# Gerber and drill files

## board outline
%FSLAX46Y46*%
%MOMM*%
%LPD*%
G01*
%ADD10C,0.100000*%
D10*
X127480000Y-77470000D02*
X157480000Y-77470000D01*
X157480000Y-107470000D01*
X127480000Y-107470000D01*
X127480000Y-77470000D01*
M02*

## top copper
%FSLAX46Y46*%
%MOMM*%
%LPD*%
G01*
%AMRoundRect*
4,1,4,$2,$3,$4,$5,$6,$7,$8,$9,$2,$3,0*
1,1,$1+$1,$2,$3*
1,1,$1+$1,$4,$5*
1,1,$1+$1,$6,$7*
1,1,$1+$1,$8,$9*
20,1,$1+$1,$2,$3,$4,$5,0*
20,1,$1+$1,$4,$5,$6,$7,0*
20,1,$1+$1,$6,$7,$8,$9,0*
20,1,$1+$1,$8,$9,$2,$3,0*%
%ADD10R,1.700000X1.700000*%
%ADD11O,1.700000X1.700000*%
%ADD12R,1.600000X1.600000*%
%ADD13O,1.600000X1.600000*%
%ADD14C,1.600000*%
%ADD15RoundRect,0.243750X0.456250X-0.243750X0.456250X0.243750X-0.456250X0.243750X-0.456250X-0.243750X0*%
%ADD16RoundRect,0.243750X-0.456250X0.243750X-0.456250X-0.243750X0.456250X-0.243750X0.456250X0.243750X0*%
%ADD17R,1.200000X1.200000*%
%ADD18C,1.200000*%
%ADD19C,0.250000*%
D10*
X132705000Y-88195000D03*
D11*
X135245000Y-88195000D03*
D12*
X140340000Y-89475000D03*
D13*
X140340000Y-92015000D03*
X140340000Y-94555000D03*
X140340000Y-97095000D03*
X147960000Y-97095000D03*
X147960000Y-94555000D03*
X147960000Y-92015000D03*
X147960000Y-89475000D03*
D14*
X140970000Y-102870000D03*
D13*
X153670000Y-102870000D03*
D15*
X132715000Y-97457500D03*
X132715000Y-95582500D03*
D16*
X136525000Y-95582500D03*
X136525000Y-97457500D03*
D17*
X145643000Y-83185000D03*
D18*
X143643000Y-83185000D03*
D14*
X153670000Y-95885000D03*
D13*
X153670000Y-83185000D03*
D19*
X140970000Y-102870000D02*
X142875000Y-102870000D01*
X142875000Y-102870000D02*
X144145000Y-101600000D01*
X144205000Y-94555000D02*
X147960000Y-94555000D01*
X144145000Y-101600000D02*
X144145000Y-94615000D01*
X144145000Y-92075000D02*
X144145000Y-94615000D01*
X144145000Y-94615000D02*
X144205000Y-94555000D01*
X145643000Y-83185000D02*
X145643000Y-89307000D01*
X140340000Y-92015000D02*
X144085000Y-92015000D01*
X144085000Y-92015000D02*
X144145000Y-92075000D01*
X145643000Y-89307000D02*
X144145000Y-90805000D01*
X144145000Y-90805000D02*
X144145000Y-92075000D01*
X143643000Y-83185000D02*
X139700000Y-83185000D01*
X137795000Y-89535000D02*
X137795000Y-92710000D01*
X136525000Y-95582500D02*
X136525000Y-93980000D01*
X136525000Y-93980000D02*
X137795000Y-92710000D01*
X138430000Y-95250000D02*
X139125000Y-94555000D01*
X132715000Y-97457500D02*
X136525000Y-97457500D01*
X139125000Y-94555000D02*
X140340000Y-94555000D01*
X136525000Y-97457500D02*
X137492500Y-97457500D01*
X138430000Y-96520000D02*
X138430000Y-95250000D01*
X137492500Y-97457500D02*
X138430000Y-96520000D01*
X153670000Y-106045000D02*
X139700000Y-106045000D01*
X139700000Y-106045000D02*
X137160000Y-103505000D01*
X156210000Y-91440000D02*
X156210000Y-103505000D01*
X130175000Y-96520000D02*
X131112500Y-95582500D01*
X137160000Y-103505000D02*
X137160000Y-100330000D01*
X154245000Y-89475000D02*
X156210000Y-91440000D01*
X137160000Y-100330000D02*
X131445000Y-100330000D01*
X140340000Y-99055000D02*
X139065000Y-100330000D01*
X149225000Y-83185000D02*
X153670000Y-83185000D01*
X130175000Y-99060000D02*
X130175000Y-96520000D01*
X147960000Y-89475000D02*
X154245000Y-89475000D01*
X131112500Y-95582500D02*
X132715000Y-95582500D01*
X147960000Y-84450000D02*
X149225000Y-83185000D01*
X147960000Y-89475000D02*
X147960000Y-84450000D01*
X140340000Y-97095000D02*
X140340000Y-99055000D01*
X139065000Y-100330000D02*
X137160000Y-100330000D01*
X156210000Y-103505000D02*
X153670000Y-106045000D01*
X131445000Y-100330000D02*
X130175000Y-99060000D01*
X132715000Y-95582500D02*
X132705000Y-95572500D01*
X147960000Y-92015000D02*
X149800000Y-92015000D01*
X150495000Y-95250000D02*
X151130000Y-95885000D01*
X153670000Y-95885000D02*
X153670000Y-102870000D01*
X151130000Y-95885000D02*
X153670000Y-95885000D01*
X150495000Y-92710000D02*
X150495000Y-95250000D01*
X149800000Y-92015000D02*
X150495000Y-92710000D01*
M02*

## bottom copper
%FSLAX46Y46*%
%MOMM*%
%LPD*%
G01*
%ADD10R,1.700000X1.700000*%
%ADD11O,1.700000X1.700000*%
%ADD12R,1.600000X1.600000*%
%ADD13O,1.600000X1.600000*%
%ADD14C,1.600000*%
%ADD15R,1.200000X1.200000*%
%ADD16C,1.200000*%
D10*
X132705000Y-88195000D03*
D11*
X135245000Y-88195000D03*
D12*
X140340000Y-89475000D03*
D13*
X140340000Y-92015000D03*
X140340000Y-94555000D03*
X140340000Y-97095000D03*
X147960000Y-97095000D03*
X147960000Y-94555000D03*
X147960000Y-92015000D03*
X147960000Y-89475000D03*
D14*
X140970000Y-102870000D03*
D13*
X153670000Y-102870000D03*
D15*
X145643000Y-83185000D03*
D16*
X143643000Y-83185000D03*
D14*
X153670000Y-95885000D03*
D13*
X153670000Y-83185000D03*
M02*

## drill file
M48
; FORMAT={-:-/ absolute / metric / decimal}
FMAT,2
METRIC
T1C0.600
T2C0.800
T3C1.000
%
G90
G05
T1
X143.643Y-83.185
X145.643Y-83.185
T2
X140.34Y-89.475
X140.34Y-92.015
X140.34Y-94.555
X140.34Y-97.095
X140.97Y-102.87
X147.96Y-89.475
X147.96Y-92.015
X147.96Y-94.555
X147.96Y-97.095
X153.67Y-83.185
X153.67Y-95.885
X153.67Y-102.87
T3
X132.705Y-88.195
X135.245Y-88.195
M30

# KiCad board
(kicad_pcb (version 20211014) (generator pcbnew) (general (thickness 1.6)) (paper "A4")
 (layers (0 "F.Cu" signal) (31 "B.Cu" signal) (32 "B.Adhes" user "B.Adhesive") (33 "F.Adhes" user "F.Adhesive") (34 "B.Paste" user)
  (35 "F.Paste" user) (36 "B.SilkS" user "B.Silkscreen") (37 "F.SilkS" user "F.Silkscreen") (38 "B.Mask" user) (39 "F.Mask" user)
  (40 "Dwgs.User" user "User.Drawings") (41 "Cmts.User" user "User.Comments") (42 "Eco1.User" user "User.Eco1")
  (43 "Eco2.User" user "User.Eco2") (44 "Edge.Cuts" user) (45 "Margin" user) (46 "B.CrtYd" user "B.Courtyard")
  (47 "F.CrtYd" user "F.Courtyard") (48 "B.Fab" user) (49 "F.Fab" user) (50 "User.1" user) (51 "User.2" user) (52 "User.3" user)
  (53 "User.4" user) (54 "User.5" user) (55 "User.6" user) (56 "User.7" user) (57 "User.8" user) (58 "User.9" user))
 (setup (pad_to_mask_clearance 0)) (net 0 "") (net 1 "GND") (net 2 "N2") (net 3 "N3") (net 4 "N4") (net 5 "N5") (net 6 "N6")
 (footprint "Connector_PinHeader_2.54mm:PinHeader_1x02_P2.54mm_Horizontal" (layer "F.Cu") (at 132.705 88.195 90)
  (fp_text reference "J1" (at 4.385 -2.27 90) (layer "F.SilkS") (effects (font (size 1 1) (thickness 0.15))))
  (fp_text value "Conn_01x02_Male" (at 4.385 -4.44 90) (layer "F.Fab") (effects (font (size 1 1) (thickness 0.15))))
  (pad "1" thru_hole rect (at 0 0 90) (size 1.7 1.7) (drill 1) (layers *.Cu *.Mask) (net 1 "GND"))
  (pad "2" thru_hole oval (at 0 2.54 90) (size 1.7 1.7) (drill 1) (layers *.Cu *.Mask) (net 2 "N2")))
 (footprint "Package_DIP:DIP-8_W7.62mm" (layer "F.Cu") (at 140.34 89.475)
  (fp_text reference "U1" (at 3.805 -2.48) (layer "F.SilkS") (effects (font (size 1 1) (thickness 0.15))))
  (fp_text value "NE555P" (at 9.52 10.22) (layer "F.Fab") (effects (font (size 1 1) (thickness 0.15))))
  (pad "1" thru_hole rect (at 0 0) (size 1.6 1.6) (drill 0.8) (layers *.Cu *.Mask) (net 1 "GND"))
  (pad "2" thru_hole oval (at 0 2.54) (size 1.6 1.6) (drill 0.8) (layers *.Cu *.Mask) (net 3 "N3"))
  (pad "3" thru_hole oval (at 0 5.08) (size 1.6 1.6) (drill 0.8) (layers *.Cu *.Mask) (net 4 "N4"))
  (pad "4" thru_hole oval (at 0 7.62) (size 1.6 1.6) (drill 0.8) (layers *.Cu *.Mask) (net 2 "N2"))
  (pad "5" thru_hole oval (at 7.62 7.62) (size 1.6 1.6) (drill 0.8) (layers *.Cu *.Mask) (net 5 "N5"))
  (pad "6" thru_hole oval (at 7.62 5.08) (size 1.6 1.6) (drill 0.8) (layers *.Cu *.Mask) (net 3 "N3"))
  (pad "7" thru_hole oval (at 7.62 2.54) (size 1.6 1.6) (drill 0.8) (layers *.Cu *.Mask) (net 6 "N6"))
  (pad "8" thru_hole oval (at 7.62 0) (size 1.6 1.6) (drill 0.8) (layers *.Cu *.Mask) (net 2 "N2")))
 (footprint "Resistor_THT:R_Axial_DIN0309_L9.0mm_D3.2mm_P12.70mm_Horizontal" (layer "F.Cu") (at 140.97 102.87)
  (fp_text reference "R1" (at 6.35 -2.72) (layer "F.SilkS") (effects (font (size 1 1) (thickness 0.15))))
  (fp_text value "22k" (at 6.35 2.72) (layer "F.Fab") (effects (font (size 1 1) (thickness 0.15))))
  (pad "1" thru_hole circle (at 0 0) (size 1.6 1.6) (drill 0.8) (layers *.Cu *.Mask) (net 3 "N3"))
  (pad "2" thru_hole oval (at 12.7 0) (size 1.6 1.6) (drill 0.8) (layers *.Cu *.Mask) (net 6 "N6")))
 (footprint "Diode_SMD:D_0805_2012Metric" (layer "F.Cu") (at 132.715 96.52 90)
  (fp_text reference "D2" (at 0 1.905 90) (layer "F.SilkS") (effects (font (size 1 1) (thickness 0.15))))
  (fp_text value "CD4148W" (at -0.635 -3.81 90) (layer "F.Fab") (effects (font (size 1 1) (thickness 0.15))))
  (pad "1" smd roundrect (at -0.9375 0 90) (size 0.975 1.4) (layers "F.Cu" "F.Paste" "F.Mask") (roundrect_rratio 0.25) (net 4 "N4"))
  (pad "2" smd roundrect (at 0.9375 0 90) (size 0.975 1.4) (layers "F.Cu" "F.Paste" "F.Mask") (roundrect_rratio 0.25) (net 2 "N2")))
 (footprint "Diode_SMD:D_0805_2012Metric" (layer "F.Cu") (at 136.525 96.52 -90)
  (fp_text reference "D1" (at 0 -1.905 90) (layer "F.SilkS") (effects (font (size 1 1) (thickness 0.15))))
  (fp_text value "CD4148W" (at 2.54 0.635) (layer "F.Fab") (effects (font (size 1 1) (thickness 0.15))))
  (pad "1" smd roundrect (at -0.9375 0 270) (size 0.975 1.4) (layers "F.Cu" "F.Paste" "F.Mask") (roundrect_rratio 0.25) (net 1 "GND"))
  (pad "2" smd roundrect (at 0.9375 0 270) (size 0.975 1.4) (layers "F.Cu" "F.Paste" "F.Mask") (roundrect_rratio 0.25) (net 4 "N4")))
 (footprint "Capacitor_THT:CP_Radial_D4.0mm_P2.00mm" (layer "F.Cu") (at 145.643 83.185 180)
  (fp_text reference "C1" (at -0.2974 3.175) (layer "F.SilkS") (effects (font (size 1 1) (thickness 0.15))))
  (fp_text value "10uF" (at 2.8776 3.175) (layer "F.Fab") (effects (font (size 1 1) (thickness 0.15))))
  (pad "1" thru_hole rect (at 0 0 180) (size 1.2 1.2) (drill 0.6) (layers *.Cu *.Mask) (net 3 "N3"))
  (pad "2" thru_hole circle (at 2 0 180) (size 1.2 1.2) (drill 0.6) (layers *.Cu *.Mask) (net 1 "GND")))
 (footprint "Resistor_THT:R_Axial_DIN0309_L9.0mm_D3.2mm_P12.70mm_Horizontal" (layer "F.Cu") (at 153.67 95.885 90)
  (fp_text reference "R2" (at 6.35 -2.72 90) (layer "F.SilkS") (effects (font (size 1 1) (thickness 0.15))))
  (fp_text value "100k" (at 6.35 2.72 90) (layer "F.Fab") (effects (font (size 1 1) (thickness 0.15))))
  (pad "1" thru_hole circle (at 0 0 90) (size 1.6 1.6) (drill 0.8) (layers *.Cu *.Mask) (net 6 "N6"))
  (pad "2" thru_hole oval (at 12.7 0 90) (size 1.6 1.6) (drill 0.8) (layers *.Cu *.Mask) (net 2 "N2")))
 (gr_rect (start 127.48 77.47) (end 157.48 107.47) (layer "Edge.Cuts") (width 0.1) (fill none))
 (segment (start 140.97 102.87) (end 142.875 102.87) (width 0.25) (layer "F.Cu") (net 3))
 (segment (start 142.875 102.87) (end 144.145 101.6) (width 0.25) (layer "F.Cu") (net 3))
 (segment (start 144.205 94.555) (end 147.96 94.555) (width 0.25) (layer "F.Cu") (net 3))
 (segment (start 144.145 101.6) (end 144.145 94.615) (width 0.25) (layer "F.Cu") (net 3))
 (segment (start 144.145 92.075) (end 144.145 94.615) (width 0.25) (layer "F.Cu") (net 3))
 (segment (start 144.145 94.615) (end 144.205 94.555) (width 0.25) (layer "F.Cu") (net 3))
 (segment (start 145.643 83.185) (end 145.643 89.307) (width 0.25) (layer "F.Cu") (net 3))
 (segment (start 140.34 92.015) (end 144.085 92.015) (width 0.25) (layer "F.Cu") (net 3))
 (segment (start 144.085 92.015) (end 144.145 92.075) (width 0.25) (layer "F.Cu") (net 3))
 (segment (start 145.643 89.307) (end 144.145 90.805) (width 0.25) (layer "F.Cu") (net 3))
 (segment (start 144.145 90.805) (end 144.145 92.075) (width 0.25) (layer "F.Cu") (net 3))
 (segment (start 143.643 83.185) (end 139.7 83.185) (width 0.25) (layer "F.Cu") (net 1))
 (segment (start 137.795 89.535) (end 137.795 92.71) (width 0.25) (layer "F.Cu") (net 1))
 (segment (start 136.525 95.5825) (end 136.525 93.98) (width 0.25) (layer "F.Cu") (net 1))
 (segment (start 136.525 93.98) (end 137.795 92.71) (width 0.25) (layer "F.Cu") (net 1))
 (segment (start 138.43 95.25) (end 139.125 94.555) (width 0.25) (layer "F.Cu") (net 4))
 (segment (start 132.715 97.4575) (end 136.525 97.4575) (width 0.25) (layer "F.Cu") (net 4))
 (segment (start 139.125 94.555) (end 140.34 94.555) (width 0.25) (layer "F.Cu") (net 4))
 (segment (start 136.525 97.4575) (end 137.4925 97.4575) (width 0.25) (layer "F.Cu") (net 4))
 (segment (start 138.43 96.52) (end 138.43 95.25) (width 0.25) (layer "F.Cu") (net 4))
 (segment (start 137.4925 97.4575) (end 138.43 96.52) (width 0.25) (layer "F.Cu") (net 4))
 (segment (start 153.67 106.045) (end 139.7 106.045) (width 0.25) (layer "F.Cu") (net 2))
 (segment (start 139.7 106.045) (end 137.16 103.505) (width 0.25) (layer "F.Cu") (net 2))
 (segment (start 156.21 91.44) (end 156.21 103.505) (width 0.25) (layer "F.Cu") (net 2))
 (segment (start 130.175 96.52) (end 131.1125 95.5825) (width 0.25) (layer "F.Cu") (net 2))
 (segment (start 137.16 103.505) (end 137.16 100.33) (width 0.25) (layer "F.Cu") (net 2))
 (segment (start 154.245 89.475) (end 156.21 91.44) (width 0.25) (layer "F.Cu") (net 2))
 (segment (start 137.16 100.33) (end 131.445 100.33) (width 0.25) (layer "F.Cu") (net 2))
 (segment (start 140.34 99.055) (end 139.065 100.33) (width 0.25) (layer "F.Cu") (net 2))
 (segment (start 149.225 83.185) (end 153.67 83.185) (width 0.25) (layer "F.Cu") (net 2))
 (segment (start 130.175 99.06) (end 130.175 96.52) (width 0.25) (layer "F.Cu") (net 2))
 (segment (start 147.96 89.475) (end 154.245 89.475) (width 0.25) (layer "F.Cu") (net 2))
 (segment (start 131.1125 95.5825) (end 132.715 95.5825) (width 0.25) (layer "F.Cu") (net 2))
 (segment (start 147.96 84.45) (end 149.225 83.185) (width 0.25) (layer "F.Cu") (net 2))
 (segment (start 147.96 89.475) (end 147.96 84.45) (width 0.25) (layer "F.Cu") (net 2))
 (segment (start 140.34 97.095) (end 140.34 99.055) (width 0.25) (layer "F.Cu") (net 2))
 (segment (start 139.065 100.33) (end 137.16 100.33) (width 0.25) (layer "F.Cu") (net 2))
 (segment (start 156.21 103.505) (end 153.67 106.045) (width 0.25) (layer "F.Cu") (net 2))
 (segment (start 131.445 100.33) (end 130.175 99.06) (width 0.25) (layer "F.Cu") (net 2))
 (segment (start 132.715 95.5825) (end 132.705 95.5725) (width 0.25) (layer "F.Cu") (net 2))
 (segment (start 147.96 92.015) (end 149.8 92.015) (width 0.25) (layer "F.Cu") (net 6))
 (segment (start 150.495 95.25) (end 151.13 95.885) (width 0.25) (layer "F.Cu") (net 6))
 (segment (start 153.67 95.885) (end 153.67 102.87) (width 0.25) (layer "F.Cu") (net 6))
 (segment (start 151.13 95.885) (end 153.67 95.885) (width 0.25) (layer "F.Cu") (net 6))
 (segment (start 150.495 92.71) (end 150.495 95.25) (width 0.25) (layer "F.Cu") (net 6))
 (segment (start 149.8 92.015) (end 150.495 92.71) (width 0.25) (layer "F.Cu") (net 6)))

